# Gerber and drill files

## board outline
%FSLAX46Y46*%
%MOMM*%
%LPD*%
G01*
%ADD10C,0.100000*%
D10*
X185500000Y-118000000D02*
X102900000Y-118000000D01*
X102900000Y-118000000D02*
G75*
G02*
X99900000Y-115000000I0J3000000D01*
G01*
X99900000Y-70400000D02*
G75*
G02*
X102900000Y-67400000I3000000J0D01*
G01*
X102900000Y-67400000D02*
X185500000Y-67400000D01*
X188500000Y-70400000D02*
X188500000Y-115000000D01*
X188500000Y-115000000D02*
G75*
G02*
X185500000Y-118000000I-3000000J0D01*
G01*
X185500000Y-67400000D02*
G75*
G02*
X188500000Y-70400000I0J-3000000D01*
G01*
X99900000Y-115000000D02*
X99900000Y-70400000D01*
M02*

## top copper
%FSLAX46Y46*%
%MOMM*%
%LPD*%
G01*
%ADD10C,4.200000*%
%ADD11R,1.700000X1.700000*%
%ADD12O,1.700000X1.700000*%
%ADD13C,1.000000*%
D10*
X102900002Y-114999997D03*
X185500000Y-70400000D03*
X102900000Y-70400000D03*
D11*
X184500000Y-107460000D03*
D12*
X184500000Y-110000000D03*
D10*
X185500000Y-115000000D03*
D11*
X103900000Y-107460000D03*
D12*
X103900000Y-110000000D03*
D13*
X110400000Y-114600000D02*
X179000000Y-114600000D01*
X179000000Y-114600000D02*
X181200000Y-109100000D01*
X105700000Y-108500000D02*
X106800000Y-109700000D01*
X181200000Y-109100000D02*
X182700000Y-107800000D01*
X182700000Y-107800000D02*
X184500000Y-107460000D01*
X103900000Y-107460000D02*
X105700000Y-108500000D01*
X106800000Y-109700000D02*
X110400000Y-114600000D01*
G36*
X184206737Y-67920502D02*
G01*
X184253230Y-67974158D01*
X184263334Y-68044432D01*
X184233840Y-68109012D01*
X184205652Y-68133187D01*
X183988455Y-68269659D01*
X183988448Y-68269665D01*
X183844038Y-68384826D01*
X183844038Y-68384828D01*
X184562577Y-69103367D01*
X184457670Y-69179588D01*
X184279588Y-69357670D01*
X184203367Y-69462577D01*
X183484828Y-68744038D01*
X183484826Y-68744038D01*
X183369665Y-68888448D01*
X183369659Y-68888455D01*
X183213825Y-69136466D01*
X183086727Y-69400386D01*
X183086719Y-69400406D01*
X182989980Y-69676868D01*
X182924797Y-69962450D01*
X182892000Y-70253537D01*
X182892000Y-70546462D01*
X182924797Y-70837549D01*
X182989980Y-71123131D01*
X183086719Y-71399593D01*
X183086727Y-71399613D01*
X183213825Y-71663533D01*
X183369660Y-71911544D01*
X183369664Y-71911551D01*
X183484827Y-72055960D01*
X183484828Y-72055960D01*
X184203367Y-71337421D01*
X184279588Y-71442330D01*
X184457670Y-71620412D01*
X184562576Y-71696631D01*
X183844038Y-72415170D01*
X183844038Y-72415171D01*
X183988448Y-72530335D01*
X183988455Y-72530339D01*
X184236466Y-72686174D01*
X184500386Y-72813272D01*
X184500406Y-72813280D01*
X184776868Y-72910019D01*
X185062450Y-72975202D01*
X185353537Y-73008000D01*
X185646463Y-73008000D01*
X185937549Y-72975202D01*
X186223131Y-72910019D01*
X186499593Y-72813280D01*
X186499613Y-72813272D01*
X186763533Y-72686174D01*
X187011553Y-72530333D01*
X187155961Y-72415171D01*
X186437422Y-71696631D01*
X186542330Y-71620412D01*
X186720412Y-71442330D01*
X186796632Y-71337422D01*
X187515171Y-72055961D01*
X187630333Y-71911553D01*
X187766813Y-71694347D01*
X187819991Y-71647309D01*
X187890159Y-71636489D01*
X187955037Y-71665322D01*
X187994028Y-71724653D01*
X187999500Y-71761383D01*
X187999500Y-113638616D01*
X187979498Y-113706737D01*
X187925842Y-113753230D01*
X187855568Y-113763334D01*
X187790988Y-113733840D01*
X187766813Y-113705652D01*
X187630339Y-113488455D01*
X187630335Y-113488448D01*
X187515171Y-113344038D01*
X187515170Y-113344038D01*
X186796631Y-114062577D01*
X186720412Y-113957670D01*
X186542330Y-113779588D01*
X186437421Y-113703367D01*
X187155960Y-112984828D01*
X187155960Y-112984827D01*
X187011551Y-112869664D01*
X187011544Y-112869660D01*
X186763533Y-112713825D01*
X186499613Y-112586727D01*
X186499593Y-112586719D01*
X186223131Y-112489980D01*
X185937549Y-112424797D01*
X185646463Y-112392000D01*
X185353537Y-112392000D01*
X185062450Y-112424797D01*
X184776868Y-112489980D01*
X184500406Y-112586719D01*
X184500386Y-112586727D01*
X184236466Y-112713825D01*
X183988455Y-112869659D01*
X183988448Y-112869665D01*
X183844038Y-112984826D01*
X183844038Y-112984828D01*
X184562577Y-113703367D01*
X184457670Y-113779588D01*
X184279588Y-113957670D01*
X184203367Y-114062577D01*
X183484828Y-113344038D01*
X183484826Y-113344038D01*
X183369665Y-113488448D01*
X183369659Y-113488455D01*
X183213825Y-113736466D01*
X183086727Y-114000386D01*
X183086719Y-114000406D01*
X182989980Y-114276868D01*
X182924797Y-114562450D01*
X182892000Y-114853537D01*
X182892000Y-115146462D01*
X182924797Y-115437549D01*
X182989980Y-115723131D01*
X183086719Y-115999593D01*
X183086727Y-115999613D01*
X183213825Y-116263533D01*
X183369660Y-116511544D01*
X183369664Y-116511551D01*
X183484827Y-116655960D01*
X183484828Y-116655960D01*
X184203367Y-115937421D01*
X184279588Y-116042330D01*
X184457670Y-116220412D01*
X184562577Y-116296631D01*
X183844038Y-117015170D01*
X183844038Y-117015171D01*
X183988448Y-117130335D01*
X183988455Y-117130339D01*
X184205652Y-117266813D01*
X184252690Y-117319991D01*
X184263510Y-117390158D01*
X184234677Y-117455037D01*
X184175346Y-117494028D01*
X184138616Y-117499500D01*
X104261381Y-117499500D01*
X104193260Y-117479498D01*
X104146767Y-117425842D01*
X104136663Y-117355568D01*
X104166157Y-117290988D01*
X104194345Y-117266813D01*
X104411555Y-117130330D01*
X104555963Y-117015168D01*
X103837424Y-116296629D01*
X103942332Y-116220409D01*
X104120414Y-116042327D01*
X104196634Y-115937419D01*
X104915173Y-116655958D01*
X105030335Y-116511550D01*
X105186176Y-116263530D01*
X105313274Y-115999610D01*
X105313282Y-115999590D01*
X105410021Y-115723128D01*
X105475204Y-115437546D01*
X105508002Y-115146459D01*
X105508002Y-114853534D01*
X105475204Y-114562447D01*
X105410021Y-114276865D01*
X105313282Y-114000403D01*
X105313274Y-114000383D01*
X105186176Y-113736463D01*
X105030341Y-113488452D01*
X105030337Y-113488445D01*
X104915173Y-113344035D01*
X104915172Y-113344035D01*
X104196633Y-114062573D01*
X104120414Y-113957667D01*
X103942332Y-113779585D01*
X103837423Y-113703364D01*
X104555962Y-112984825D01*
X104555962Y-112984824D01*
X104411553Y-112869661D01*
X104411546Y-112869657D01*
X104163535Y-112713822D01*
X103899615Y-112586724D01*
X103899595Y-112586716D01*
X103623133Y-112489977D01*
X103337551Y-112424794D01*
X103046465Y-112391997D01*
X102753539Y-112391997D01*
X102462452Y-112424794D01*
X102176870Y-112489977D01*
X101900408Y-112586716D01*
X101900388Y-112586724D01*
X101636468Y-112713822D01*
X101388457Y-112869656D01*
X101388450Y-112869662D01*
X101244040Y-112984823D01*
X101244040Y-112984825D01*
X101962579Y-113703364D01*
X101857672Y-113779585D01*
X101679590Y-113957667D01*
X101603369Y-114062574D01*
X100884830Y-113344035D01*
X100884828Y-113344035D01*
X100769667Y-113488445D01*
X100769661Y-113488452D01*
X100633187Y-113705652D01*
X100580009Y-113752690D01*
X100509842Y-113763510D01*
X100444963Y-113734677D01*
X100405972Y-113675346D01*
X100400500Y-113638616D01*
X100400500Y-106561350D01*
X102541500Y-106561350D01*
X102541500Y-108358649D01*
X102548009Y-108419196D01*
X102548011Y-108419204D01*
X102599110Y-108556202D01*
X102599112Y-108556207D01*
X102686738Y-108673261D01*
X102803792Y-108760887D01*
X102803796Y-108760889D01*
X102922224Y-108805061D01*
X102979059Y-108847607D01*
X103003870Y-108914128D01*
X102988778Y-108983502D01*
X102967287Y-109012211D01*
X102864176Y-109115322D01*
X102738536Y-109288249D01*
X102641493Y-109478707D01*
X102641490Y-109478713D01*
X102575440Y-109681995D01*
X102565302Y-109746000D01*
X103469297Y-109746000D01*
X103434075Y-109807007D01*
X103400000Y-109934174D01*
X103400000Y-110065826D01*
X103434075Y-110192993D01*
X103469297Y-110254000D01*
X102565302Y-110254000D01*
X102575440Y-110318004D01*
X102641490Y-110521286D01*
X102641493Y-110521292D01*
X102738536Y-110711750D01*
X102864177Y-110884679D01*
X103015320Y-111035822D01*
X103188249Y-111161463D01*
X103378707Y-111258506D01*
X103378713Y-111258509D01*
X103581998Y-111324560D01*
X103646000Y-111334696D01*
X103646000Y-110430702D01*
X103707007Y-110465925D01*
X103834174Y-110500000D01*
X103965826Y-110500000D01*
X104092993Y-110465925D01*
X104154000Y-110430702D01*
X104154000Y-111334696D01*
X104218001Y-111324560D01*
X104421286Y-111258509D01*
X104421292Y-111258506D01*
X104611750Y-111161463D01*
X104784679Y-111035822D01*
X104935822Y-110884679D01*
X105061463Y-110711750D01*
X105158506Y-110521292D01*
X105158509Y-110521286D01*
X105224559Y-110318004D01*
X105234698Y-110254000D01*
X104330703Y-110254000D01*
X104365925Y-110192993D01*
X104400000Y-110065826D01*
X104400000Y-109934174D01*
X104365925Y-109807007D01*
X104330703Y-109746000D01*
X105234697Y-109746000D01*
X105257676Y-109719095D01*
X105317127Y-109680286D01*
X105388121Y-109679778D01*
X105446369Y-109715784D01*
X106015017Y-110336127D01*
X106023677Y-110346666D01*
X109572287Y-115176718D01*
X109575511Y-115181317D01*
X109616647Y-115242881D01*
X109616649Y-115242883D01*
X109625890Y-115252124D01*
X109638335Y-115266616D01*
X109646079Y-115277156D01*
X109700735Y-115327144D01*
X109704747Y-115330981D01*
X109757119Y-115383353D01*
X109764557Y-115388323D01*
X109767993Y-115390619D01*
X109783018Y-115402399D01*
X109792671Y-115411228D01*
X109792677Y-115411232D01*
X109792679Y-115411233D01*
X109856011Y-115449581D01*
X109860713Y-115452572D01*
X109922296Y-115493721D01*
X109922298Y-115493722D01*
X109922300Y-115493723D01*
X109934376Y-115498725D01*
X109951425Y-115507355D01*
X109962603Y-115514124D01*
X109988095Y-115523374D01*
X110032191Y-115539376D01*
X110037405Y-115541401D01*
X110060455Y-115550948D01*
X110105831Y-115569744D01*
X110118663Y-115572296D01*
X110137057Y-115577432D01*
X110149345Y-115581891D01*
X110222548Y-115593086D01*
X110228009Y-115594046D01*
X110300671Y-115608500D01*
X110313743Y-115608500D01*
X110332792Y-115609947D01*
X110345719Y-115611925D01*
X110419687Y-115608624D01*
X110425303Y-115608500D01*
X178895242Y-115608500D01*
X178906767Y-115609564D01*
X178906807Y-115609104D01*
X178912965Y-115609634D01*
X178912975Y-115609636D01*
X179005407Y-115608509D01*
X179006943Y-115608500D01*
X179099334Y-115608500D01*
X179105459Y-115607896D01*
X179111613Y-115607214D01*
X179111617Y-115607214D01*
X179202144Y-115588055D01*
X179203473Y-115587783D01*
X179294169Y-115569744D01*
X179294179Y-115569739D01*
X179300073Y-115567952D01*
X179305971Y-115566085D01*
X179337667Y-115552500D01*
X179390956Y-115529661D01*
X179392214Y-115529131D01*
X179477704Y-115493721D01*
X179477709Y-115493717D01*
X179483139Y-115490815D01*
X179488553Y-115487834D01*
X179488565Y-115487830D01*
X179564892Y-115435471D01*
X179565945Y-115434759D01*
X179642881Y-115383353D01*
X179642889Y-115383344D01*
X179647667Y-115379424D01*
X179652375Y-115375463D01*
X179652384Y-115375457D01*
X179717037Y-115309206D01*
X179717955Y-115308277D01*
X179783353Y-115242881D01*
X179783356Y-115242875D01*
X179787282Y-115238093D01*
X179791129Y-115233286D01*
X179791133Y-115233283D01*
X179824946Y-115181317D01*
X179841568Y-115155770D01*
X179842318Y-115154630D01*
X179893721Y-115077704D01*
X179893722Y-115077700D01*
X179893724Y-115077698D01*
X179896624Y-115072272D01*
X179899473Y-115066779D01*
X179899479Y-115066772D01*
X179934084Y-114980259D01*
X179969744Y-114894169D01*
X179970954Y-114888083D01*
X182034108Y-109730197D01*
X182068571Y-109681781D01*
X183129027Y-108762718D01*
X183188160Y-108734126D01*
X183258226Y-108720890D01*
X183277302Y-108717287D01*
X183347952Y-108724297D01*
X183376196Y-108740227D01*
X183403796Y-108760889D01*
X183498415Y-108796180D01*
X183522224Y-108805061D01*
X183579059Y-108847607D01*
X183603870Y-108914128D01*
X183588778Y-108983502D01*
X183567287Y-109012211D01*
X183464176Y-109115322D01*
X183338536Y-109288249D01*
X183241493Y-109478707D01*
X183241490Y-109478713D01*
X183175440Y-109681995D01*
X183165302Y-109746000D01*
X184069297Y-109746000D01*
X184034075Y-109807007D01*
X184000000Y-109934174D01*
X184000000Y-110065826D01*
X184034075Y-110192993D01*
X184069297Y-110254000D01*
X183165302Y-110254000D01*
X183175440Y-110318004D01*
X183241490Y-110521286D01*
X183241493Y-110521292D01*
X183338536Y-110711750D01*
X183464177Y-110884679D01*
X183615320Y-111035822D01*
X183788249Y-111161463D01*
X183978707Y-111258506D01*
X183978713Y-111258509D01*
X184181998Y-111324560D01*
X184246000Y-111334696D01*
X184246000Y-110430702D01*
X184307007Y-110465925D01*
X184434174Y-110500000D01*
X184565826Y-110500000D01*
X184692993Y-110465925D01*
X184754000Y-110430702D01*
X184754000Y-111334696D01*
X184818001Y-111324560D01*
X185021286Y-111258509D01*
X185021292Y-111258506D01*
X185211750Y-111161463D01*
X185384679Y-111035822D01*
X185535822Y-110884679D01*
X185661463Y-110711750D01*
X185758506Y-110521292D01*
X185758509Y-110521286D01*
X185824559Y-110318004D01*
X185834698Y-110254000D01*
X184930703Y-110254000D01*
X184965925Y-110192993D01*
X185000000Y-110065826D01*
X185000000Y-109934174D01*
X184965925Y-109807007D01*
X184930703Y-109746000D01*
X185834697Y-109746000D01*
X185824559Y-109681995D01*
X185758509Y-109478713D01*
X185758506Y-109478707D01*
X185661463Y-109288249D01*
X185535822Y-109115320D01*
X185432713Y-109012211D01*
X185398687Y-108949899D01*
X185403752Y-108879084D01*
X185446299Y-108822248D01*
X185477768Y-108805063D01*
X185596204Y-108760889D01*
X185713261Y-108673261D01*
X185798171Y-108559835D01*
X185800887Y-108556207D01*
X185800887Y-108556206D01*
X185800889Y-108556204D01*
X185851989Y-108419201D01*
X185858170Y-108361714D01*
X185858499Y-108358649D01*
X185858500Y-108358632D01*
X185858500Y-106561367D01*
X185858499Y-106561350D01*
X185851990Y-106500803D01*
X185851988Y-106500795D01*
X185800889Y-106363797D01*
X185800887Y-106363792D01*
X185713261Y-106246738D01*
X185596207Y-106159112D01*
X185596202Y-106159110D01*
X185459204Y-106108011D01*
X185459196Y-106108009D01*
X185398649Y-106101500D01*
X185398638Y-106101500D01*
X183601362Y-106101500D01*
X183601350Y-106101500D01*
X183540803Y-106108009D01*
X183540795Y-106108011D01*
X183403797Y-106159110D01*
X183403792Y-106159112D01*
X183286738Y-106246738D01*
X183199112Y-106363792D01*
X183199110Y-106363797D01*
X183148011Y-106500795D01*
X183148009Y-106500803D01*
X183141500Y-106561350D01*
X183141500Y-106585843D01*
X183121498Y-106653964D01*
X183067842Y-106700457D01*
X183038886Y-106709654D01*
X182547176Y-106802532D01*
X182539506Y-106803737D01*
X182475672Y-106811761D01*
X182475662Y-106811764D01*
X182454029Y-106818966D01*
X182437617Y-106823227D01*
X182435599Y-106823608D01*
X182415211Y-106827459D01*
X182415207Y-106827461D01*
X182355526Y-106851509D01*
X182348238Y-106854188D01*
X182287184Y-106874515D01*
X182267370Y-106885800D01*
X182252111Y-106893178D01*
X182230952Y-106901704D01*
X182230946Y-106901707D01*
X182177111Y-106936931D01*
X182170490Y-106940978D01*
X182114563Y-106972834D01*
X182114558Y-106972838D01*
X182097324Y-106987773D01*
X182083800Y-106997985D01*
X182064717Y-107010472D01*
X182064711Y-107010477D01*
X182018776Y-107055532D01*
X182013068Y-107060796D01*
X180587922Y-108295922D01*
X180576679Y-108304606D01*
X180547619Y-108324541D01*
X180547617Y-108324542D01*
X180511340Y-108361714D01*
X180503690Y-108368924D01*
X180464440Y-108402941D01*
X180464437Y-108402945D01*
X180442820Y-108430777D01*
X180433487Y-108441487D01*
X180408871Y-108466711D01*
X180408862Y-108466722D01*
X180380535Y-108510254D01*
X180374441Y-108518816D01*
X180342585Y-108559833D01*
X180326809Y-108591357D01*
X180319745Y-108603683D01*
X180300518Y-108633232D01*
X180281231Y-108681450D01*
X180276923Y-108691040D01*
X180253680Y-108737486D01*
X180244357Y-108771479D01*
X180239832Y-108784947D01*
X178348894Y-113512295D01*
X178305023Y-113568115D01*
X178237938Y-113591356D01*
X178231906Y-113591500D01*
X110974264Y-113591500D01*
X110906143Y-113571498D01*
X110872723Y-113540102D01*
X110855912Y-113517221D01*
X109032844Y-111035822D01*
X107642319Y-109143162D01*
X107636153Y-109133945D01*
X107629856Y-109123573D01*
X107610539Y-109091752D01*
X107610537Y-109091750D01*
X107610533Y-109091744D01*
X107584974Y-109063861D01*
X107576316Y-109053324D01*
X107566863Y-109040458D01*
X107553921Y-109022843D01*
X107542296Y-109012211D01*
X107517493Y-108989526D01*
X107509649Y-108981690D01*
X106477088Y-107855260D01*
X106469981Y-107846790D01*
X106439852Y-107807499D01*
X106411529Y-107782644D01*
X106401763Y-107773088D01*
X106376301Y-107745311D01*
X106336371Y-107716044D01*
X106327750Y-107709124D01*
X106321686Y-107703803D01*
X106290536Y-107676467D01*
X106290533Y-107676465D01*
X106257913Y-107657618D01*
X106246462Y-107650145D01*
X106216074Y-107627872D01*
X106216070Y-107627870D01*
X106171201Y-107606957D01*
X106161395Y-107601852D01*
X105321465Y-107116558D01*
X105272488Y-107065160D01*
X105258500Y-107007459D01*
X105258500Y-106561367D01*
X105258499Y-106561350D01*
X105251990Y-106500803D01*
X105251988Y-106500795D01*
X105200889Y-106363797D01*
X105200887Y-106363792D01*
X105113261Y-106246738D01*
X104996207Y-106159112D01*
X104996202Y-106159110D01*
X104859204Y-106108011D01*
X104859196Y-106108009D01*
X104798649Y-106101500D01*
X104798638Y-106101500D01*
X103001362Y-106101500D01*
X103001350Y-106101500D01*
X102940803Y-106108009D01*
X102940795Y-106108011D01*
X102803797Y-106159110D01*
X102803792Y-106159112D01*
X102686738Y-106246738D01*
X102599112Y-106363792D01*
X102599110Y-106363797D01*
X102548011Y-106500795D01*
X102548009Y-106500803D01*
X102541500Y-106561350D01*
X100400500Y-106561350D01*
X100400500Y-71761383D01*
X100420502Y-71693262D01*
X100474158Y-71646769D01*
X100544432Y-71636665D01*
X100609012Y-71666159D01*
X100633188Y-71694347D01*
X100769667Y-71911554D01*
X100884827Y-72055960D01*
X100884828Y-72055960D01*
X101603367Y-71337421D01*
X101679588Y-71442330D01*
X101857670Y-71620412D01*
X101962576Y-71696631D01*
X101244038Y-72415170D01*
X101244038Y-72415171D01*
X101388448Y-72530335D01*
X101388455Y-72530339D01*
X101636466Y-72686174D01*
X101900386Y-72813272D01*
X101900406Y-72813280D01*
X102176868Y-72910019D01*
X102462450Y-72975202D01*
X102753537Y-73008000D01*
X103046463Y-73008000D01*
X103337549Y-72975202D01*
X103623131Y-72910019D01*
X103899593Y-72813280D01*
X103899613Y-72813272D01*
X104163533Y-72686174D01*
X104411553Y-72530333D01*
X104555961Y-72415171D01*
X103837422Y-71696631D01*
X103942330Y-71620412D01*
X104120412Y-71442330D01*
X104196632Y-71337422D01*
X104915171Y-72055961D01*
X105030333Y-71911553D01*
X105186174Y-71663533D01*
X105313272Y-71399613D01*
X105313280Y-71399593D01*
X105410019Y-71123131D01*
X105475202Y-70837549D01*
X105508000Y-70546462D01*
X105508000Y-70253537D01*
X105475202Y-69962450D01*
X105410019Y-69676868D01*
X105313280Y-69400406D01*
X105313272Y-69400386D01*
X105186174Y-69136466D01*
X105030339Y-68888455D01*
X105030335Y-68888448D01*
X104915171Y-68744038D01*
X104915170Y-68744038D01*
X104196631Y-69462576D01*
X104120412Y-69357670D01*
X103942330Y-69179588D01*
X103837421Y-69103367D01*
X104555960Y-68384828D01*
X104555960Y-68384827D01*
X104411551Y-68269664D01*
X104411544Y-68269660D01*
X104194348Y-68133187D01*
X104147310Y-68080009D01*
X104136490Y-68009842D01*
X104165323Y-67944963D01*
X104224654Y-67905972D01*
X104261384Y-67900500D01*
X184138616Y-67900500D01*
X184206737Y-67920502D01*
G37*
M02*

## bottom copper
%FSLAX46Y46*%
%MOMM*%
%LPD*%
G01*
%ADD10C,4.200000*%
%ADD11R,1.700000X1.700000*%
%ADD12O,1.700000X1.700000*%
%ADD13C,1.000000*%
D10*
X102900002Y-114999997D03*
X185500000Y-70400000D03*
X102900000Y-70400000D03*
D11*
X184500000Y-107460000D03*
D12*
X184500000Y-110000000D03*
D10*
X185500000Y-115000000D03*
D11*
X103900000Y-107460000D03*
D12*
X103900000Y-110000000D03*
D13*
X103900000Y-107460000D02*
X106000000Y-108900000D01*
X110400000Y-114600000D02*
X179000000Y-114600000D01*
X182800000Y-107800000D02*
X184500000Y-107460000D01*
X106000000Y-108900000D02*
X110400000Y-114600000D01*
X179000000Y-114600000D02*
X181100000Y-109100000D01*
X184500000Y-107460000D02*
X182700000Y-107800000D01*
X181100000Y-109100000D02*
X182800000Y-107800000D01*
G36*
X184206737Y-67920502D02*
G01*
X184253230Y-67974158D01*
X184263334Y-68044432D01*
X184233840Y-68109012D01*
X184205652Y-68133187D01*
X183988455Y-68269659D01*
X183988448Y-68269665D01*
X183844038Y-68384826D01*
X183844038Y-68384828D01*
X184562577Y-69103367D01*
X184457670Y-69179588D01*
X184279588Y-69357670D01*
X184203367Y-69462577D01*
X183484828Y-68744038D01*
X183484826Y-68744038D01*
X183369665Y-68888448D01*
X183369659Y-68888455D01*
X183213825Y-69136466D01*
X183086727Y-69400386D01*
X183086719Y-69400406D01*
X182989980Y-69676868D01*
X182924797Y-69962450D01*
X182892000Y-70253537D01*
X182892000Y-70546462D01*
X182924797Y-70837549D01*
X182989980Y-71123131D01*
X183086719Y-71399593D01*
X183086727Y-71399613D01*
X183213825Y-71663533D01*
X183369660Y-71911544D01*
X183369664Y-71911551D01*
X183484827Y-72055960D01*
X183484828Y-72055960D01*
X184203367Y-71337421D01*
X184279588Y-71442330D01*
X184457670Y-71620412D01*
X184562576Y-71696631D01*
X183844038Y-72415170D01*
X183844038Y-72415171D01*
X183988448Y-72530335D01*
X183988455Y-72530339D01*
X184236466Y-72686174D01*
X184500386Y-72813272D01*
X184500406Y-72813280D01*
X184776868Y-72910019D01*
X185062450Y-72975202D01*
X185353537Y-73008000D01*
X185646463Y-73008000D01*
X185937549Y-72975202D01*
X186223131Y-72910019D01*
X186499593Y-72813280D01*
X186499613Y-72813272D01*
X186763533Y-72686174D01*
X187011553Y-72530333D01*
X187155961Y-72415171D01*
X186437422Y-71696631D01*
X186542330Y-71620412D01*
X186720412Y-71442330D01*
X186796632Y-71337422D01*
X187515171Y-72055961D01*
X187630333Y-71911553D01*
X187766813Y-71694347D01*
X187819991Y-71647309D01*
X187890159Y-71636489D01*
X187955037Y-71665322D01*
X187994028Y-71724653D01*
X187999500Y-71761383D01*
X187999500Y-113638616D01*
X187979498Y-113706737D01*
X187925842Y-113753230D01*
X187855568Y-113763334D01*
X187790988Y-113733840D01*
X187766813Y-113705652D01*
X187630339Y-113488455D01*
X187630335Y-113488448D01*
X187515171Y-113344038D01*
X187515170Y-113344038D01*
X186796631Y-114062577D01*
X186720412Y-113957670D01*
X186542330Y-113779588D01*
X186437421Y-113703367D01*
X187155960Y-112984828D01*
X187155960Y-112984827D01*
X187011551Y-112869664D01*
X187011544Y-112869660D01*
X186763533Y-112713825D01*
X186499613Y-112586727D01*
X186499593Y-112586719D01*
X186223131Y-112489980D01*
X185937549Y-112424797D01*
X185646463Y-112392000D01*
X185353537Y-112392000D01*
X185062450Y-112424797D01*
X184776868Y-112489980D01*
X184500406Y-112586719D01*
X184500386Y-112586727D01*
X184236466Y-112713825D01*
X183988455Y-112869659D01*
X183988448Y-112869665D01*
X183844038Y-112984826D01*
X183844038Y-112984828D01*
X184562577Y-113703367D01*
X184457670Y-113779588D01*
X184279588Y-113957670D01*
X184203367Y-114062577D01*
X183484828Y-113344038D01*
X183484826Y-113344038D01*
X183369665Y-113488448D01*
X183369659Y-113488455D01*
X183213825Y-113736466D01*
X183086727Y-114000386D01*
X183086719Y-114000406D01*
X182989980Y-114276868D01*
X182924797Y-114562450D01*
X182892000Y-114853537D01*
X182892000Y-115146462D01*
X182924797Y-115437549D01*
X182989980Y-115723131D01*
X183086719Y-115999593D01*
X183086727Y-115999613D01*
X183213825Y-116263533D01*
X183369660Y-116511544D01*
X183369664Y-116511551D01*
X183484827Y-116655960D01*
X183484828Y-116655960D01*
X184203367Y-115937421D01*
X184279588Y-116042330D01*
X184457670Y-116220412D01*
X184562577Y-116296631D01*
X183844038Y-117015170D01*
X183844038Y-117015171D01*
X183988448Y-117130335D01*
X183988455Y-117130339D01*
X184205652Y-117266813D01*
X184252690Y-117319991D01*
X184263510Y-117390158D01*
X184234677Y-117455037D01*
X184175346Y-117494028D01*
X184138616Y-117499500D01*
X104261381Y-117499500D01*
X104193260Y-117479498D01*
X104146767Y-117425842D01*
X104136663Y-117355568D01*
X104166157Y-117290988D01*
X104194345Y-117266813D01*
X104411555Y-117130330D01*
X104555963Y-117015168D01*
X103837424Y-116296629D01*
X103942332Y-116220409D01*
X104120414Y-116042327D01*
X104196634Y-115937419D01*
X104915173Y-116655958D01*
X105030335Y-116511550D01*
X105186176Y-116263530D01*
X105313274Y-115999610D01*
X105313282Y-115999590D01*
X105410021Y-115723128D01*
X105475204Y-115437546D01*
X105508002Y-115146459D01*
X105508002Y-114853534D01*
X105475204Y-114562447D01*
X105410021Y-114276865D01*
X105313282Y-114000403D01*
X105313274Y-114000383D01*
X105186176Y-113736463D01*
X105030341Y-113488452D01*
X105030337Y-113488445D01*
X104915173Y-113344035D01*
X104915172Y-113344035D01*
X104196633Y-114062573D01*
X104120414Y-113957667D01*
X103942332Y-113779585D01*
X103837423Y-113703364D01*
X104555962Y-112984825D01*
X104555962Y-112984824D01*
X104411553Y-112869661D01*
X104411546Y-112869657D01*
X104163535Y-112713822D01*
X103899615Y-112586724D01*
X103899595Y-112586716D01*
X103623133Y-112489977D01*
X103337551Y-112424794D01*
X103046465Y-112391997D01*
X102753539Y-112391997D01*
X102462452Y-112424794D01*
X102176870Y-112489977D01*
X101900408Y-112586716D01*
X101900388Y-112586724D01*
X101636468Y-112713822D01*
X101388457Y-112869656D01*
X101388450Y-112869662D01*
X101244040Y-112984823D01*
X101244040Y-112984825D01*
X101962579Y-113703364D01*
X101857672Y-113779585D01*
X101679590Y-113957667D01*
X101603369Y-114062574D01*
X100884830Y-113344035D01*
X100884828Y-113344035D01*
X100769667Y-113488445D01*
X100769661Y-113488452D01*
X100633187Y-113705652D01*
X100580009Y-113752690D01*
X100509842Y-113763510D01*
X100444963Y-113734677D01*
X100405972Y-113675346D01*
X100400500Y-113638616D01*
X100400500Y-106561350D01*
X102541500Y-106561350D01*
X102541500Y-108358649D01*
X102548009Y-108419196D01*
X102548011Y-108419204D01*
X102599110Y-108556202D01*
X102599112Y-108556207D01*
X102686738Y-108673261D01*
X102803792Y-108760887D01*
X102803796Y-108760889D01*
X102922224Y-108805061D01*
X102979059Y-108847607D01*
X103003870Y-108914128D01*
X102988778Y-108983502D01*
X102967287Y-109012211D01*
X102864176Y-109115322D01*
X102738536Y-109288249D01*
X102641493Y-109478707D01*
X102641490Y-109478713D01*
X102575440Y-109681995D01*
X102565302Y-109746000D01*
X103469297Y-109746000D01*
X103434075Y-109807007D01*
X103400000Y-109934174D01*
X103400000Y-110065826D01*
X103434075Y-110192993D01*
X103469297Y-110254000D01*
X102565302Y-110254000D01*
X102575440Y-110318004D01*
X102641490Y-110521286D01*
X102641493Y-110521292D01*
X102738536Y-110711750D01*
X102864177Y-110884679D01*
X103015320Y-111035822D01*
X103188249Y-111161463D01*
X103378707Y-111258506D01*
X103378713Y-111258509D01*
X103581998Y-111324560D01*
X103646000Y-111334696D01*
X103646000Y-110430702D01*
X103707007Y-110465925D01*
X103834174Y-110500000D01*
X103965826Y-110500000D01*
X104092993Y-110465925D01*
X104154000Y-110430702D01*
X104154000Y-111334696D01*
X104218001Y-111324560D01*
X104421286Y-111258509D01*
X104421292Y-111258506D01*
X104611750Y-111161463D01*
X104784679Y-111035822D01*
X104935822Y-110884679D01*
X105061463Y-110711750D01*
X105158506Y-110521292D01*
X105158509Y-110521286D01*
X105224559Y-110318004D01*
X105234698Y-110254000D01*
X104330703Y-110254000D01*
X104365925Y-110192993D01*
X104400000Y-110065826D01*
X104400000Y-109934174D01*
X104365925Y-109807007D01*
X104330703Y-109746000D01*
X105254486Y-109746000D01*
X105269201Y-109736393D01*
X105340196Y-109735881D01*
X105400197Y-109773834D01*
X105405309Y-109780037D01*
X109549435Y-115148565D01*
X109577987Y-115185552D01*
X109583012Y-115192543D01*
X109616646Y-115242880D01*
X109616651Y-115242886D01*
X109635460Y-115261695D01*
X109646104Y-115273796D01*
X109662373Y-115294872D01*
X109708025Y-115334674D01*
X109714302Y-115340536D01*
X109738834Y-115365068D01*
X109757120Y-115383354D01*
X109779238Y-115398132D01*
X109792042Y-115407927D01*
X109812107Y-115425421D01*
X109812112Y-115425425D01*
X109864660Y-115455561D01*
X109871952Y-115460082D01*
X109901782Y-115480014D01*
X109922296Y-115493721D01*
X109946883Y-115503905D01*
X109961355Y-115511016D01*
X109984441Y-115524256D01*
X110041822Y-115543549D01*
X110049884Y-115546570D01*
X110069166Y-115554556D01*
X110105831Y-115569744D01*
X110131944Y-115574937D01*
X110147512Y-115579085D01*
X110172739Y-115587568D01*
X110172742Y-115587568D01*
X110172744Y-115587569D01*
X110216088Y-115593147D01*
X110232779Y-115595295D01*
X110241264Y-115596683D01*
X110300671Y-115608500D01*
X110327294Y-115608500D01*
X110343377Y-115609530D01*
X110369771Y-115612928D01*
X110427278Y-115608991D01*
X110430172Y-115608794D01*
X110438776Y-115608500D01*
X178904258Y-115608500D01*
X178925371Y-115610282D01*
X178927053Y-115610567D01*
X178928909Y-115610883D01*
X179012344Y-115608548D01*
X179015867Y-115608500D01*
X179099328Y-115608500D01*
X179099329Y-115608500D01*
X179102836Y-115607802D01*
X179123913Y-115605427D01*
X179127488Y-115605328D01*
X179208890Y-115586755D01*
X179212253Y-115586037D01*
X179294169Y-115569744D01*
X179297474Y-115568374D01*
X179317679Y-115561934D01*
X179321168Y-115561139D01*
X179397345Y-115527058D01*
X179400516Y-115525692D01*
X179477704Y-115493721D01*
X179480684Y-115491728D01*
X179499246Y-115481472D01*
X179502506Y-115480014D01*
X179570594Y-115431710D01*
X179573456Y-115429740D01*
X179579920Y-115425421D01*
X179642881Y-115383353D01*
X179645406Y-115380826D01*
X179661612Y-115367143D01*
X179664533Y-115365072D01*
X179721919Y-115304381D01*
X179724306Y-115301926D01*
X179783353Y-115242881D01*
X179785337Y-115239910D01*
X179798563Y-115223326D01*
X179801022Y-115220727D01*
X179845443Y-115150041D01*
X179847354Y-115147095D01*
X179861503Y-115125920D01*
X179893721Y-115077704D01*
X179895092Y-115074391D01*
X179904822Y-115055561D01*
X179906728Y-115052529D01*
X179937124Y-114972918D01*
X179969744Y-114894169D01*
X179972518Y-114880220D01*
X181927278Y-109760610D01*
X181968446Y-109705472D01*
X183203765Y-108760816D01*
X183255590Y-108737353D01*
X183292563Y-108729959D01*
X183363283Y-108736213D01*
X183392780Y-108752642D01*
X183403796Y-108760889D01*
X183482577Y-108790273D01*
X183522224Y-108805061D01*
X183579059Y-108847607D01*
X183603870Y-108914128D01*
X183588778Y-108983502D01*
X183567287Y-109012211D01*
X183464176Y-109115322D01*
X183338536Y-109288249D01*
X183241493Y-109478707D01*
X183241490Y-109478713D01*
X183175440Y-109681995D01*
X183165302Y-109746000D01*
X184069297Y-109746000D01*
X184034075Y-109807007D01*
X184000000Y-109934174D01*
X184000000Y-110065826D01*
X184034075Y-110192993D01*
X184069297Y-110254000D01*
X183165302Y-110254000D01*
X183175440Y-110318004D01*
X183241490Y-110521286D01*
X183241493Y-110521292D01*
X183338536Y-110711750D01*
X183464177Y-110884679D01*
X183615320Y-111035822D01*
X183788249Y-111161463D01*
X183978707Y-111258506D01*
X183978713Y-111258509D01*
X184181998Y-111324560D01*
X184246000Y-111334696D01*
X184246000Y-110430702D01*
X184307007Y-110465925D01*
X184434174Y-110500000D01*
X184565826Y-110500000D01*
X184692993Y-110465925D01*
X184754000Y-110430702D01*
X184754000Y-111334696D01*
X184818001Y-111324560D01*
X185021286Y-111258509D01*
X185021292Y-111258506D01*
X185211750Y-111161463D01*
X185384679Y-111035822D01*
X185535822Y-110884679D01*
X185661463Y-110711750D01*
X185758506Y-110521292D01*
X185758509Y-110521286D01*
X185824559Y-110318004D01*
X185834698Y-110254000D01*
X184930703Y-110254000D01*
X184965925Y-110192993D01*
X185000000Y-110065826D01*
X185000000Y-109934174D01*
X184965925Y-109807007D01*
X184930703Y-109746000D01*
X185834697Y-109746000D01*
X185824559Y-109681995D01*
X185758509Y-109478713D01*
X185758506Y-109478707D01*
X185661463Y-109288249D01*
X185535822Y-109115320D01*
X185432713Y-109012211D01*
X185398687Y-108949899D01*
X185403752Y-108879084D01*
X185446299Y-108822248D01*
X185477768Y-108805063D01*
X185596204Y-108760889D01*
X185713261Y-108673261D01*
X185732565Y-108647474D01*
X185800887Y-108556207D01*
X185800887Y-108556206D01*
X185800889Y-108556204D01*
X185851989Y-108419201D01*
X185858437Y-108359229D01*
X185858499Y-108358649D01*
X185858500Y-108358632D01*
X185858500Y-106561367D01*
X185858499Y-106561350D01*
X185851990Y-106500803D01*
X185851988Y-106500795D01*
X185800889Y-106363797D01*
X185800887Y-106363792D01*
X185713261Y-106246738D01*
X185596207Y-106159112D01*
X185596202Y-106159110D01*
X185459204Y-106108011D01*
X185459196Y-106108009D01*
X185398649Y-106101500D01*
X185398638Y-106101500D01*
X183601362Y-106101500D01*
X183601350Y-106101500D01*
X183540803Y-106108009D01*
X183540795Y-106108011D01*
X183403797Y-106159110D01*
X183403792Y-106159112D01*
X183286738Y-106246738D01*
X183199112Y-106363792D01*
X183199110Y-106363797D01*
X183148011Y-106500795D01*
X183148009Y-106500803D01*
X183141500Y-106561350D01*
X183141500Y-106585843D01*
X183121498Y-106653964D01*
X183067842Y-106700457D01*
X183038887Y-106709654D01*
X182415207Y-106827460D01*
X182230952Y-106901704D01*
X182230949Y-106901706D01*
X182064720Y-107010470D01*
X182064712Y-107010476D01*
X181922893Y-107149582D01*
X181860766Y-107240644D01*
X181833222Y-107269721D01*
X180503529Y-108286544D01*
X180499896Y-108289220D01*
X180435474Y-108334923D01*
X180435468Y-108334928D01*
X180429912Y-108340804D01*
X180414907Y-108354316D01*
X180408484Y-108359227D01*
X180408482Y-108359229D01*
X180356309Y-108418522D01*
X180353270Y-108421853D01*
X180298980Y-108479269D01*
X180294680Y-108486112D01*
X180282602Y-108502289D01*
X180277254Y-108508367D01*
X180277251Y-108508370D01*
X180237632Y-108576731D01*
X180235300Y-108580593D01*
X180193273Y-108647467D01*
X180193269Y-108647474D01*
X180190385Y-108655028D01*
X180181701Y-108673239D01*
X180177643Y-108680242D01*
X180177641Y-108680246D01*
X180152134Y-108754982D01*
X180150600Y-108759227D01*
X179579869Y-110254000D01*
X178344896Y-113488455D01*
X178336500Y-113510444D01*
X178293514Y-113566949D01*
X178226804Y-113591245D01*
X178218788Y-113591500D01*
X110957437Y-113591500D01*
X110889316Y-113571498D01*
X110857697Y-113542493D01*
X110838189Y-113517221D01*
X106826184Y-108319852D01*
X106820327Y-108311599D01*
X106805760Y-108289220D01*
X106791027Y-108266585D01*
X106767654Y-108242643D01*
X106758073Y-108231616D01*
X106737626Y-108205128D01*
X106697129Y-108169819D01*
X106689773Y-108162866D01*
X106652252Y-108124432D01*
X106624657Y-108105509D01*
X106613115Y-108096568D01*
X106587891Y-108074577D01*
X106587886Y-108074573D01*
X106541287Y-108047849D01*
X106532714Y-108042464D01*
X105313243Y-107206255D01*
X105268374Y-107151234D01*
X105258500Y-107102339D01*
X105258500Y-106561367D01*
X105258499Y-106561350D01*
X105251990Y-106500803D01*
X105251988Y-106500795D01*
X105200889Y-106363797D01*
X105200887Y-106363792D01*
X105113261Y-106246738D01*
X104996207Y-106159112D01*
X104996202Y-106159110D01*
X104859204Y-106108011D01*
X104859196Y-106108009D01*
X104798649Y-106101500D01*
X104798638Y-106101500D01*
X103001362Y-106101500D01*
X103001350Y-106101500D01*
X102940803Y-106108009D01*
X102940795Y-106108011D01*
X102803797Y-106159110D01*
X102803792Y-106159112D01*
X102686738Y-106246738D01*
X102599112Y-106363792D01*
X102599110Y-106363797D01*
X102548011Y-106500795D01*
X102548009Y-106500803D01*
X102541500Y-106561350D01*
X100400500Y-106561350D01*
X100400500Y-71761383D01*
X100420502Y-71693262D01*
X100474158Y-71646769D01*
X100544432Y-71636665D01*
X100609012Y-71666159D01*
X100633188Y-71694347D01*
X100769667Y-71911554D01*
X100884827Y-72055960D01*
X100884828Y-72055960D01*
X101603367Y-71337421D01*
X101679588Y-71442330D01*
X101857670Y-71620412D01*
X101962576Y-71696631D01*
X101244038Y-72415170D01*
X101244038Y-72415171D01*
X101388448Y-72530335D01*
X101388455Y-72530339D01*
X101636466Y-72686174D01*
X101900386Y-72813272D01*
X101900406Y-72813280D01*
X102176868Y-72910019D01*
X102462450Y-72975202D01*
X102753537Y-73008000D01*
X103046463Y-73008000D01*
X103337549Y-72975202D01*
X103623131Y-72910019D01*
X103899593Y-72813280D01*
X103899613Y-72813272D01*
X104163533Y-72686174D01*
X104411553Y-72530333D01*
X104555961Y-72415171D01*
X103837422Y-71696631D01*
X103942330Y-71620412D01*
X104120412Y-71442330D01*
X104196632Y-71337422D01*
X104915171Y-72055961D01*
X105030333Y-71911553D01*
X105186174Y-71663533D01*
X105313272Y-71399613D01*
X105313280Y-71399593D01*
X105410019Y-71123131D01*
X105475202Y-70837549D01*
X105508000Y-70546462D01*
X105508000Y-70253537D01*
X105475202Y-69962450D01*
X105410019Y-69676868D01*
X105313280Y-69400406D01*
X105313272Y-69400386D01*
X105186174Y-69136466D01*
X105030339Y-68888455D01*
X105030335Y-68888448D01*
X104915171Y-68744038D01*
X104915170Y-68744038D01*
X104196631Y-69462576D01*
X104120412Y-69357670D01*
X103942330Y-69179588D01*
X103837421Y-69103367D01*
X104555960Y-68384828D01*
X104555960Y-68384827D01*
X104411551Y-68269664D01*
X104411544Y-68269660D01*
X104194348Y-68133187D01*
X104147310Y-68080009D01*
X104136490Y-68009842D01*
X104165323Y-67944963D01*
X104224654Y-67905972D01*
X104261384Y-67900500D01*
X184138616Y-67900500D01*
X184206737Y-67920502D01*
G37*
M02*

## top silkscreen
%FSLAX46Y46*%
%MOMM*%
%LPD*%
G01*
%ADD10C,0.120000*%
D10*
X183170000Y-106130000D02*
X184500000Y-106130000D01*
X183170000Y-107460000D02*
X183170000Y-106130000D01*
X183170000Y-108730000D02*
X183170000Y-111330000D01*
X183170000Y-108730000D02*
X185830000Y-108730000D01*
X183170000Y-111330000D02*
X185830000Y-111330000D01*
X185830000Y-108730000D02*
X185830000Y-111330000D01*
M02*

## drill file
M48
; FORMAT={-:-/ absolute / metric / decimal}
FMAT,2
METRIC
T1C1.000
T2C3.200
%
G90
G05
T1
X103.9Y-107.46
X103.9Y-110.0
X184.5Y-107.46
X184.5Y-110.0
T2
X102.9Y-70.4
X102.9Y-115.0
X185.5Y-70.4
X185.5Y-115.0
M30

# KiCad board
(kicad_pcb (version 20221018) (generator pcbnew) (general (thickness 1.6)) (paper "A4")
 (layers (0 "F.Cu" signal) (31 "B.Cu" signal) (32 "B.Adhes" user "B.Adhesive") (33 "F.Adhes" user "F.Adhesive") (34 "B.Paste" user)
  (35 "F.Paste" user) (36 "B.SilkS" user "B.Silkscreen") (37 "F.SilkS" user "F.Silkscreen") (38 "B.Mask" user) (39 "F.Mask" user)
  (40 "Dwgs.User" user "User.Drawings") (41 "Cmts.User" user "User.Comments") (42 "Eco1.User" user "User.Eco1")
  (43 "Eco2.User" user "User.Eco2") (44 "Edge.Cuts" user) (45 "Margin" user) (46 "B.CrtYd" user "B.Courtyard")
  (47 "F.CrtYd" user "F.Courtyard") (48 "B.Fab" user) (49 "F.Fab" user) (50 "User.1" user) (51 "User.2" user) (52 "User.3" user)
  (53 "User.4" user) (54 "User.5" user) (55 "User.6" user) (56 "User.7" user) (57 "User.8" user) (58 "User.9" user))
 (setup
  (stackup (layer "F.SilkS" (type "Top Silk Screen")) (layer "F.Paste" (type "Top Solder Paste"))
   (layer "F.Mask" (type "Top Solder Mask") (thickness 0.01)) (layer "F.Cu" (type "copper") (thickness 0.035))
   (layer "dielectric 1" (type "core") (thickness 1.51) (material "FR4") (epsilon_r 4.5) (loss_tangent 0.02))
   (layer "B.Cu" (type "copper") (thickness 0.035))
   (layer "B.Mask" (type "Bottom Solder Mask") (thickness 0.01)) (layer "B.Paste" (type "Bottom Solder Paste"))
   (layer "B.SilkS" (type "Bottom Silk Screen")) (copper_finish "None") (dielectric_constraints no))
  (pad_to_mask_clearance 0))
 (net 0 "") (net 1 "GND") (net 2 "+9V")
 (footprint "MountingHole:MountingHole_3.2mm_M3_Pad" (layer "F.Cu") (at 102.900002 114.999997)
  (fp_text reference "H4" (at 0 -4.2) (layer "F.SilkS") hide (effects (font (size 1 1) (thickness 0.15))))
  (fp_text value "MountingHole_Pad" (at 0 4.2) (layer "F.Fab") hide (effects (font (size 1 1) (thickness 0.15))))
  (pad "1" thru_hole circle (at 0 0) (size 4.2 4.2) (drill 3.2) (layers "*.Cu" "*.Mask") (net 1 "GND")))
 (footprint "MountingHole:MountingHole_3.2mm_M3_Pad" (layer "F.Cu") (at 185.5 70.4)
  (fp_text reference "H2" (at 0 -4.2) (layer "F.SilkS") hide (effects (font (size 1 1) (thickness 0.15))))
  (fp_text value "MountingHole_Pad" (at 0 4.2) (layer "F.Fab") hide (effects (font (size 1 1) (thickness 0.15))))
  (pad "1" thru_hole circle (at 0 0) (size 4.2 4.2) (drill 3.2) (layers "*.Cu" "*.Mask") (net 1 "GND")))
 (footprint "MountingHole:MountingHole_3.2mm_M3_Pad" (layer "F.Cu") (at 102.9 70.4)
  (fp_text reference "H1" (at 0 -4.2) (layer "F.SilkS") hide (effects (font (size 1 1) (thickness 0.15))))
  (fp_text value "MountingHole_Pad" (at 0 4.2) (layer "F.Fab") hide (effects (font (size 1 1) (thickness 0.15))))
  (pad "1" thru_hole circle (at 0 0) (size 4.2 4.2) (drill 3.2) (layers "*.Cu" "*.Mask") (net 1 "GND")))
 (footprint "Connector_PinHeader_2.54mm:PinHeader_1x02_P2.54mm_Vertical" (layer "F.Cu") (at 184.5 107.46)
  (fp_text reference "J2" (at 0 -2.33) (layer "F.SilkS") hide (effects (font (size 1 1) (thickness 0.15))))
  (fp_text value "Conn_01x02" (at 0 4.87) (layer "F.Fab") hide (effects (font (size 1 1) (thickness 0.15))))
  (fp_line (start -1.33 -1.33) (end 0 -1.33) (stroke (width 0.12) (type solid)) (layer "F.SilkS"))
  (fp_line (start -1.33 0) (end -1.33 -1.33) (stroke (width 0.12) (type solid)) (layer "F.SilkS"))
  (fp_line (start -1.33 1.27) (end -1.33 3.87) (stroke (width 0.12) (type solid)) (layer "F.SilkS"))
  (fp_line (start -1.33 1.27) (end 1.33 1.27) (stroke (width 0.12) (type solid)) (layer "F.SilkS"))
  (fp_line (start -1.33 3.87) (end 1.33 3.87) (stroke (width 0.12) (type solid)) (layer "F.SilkS"))
  (fp_line (start 1.33 1.27) (end 1.33 3.87) (stroke (width 0.12) (type solid)) (layer "F.SilkS"))
  (pad "1" thru_hole rect (at 0 0) (size 1.7 1.7) (drill 1) (layers "*.Cu" "*.Mask") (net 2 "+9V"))
  (pad "2" thru_hole oval (at 0 2.54) (size 1.7 1.7) (drill 1) (layers "*.Cu" "*.Mask") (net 1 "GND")))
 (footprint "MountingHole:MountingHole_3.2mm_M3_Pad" (layer "F.Cu") (at 185.5 115)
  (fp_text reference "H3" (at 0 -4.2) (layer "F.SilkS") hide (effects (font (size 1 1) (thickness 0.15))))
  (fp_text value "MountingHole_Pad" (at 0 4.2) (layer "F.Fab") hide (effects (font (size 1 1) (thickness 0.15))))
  (pad "1" thru_hole circle (at 0 0) (size 4.2 4.2) (drill 3.2) (layers "*.Cu" "*.Mask") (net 1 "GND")))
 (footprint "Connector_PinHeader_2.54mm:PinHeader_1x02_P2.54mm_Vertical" (layer "B.Cu") (at 103.9 107.46 180)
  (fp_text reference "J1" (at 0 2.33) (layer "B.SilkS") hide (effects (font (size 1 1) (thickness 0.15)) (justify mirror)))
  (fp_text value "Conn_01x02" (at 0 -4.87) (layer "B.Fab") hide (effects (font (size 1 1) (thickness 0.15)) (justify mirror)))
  (pad "1" thru_hole rect (at 0 0 180) (size 1.7 1.7) (drill 1) (layers "*.Cu" "*.Mask") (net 2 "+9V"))
  (pad "2" thru_hole oval (at 0 -2.54 180) (size 1.7 1.7) (drill 1) (layers "*.Cu" "*.Mask") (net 1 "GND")))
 (gr_line (start 185.5 118) (end 102.9 118) (stroke (width 0.1) (type solid)) (layer "Edge.Cuts"))
 (gr_arc (start 102.9 118) (mid 100.77868 117.12132) (end 99.9 115) (stroke (width 0.1) (type solid)) (layer "Edge.Cuts"))
 (gr_arc (start 99.9 70.4) (mid 100.778681 68.278681) (end 102.9 67.4) (stroke (width 0.1) (type solid)) (layer "Edge.Cuts"))
 (gr_line (start 102.9 67.4) (end 185.5 67.4) (stroke (width 0.1) (type solid)) (layer "Edge.Cuts"))
 (gr_line (start 188.5 70.4) (end 188.5 115) (stroke (width 0.1) (type solid)) (layer "Edge.Cuts"))
 (gr_arc (start 188.5 115) (mid 187.62132 117.12132) (end 185.5 118) (stroke (width 0.1) (type solid)) (layer "Edge.Cuts"))
 (gr_arc (start 185.5 67.4) (mid 187.621319 68.278681) (end 188.5 70.4) (stroke (width 0.1) (type solid)) (layer "Edge.Cuts"))
 (gr_line (start 99.9 115) (end 99.9 70.4) (stroke (width 0.1) (type solid)) (layer "Edge.Cuts"))
 (segment (start 110.4 114.6) (end 179 114.6) (width 1) (layer "F.Cu") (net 2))
 (segment (start 179 114.6) (end 181.2 109.1) (width 1) (layer "F.Cu") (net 2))
 (segment (start 105.7 108.5) (end 106.8 109.7) (width 1) (layer "F.Cu") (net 2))
 (segment (start 181.2 109.1) (end 182.7 107.8) (width 1) (layer "F.Cu") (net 2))
 (segment (start 182.7 107.8) (end 184.5 107.46) (width 1) (layer "F.Cu") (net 2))
 (segment (start 103.9 107.46) (end 105.7 108.5) (width 1) (layer "F.Cu") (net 2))
 (segment (start 106.8 109.7) (end 110.4 114.6) (width 1) (layer "F.Cu") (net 2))
 (segment (start 103.9 107.46) (end 106 108.9) (width 1) (layer "B.Cu") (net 2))
 (segment (start 110.4 114.6) (end 179 114.6) (width 1) (layer "B.Cu") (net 2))
 (segment (start 182.8 107.8) (end 184.5 107.46) (width 1) (layer "B.Cu") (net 2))
 (segment (start 106 108.9) (end 110.4 114.6) (width 1) (layer "B.Cu") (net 2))
 (segment (start 179 114.6) (end 181.1 109.1) (width 1) (layer "B.Cu") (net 2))
 (segment (start 184.5 107.46) (end 182.7 107.8) (width 1) (layer "B.Cu") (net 2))
 (segment (start 181.1 109.1) (end 182.8 107.8) (width 1) (layer "B.Cu") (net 2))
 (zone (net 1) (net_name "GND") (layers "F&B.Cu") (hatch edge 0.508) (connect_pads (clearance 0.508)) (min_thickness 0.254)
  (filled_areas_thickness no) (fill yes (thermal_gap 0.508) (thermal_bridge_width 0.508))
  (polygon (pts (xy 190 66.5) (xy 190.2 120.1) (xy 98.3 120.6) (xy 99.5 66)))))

